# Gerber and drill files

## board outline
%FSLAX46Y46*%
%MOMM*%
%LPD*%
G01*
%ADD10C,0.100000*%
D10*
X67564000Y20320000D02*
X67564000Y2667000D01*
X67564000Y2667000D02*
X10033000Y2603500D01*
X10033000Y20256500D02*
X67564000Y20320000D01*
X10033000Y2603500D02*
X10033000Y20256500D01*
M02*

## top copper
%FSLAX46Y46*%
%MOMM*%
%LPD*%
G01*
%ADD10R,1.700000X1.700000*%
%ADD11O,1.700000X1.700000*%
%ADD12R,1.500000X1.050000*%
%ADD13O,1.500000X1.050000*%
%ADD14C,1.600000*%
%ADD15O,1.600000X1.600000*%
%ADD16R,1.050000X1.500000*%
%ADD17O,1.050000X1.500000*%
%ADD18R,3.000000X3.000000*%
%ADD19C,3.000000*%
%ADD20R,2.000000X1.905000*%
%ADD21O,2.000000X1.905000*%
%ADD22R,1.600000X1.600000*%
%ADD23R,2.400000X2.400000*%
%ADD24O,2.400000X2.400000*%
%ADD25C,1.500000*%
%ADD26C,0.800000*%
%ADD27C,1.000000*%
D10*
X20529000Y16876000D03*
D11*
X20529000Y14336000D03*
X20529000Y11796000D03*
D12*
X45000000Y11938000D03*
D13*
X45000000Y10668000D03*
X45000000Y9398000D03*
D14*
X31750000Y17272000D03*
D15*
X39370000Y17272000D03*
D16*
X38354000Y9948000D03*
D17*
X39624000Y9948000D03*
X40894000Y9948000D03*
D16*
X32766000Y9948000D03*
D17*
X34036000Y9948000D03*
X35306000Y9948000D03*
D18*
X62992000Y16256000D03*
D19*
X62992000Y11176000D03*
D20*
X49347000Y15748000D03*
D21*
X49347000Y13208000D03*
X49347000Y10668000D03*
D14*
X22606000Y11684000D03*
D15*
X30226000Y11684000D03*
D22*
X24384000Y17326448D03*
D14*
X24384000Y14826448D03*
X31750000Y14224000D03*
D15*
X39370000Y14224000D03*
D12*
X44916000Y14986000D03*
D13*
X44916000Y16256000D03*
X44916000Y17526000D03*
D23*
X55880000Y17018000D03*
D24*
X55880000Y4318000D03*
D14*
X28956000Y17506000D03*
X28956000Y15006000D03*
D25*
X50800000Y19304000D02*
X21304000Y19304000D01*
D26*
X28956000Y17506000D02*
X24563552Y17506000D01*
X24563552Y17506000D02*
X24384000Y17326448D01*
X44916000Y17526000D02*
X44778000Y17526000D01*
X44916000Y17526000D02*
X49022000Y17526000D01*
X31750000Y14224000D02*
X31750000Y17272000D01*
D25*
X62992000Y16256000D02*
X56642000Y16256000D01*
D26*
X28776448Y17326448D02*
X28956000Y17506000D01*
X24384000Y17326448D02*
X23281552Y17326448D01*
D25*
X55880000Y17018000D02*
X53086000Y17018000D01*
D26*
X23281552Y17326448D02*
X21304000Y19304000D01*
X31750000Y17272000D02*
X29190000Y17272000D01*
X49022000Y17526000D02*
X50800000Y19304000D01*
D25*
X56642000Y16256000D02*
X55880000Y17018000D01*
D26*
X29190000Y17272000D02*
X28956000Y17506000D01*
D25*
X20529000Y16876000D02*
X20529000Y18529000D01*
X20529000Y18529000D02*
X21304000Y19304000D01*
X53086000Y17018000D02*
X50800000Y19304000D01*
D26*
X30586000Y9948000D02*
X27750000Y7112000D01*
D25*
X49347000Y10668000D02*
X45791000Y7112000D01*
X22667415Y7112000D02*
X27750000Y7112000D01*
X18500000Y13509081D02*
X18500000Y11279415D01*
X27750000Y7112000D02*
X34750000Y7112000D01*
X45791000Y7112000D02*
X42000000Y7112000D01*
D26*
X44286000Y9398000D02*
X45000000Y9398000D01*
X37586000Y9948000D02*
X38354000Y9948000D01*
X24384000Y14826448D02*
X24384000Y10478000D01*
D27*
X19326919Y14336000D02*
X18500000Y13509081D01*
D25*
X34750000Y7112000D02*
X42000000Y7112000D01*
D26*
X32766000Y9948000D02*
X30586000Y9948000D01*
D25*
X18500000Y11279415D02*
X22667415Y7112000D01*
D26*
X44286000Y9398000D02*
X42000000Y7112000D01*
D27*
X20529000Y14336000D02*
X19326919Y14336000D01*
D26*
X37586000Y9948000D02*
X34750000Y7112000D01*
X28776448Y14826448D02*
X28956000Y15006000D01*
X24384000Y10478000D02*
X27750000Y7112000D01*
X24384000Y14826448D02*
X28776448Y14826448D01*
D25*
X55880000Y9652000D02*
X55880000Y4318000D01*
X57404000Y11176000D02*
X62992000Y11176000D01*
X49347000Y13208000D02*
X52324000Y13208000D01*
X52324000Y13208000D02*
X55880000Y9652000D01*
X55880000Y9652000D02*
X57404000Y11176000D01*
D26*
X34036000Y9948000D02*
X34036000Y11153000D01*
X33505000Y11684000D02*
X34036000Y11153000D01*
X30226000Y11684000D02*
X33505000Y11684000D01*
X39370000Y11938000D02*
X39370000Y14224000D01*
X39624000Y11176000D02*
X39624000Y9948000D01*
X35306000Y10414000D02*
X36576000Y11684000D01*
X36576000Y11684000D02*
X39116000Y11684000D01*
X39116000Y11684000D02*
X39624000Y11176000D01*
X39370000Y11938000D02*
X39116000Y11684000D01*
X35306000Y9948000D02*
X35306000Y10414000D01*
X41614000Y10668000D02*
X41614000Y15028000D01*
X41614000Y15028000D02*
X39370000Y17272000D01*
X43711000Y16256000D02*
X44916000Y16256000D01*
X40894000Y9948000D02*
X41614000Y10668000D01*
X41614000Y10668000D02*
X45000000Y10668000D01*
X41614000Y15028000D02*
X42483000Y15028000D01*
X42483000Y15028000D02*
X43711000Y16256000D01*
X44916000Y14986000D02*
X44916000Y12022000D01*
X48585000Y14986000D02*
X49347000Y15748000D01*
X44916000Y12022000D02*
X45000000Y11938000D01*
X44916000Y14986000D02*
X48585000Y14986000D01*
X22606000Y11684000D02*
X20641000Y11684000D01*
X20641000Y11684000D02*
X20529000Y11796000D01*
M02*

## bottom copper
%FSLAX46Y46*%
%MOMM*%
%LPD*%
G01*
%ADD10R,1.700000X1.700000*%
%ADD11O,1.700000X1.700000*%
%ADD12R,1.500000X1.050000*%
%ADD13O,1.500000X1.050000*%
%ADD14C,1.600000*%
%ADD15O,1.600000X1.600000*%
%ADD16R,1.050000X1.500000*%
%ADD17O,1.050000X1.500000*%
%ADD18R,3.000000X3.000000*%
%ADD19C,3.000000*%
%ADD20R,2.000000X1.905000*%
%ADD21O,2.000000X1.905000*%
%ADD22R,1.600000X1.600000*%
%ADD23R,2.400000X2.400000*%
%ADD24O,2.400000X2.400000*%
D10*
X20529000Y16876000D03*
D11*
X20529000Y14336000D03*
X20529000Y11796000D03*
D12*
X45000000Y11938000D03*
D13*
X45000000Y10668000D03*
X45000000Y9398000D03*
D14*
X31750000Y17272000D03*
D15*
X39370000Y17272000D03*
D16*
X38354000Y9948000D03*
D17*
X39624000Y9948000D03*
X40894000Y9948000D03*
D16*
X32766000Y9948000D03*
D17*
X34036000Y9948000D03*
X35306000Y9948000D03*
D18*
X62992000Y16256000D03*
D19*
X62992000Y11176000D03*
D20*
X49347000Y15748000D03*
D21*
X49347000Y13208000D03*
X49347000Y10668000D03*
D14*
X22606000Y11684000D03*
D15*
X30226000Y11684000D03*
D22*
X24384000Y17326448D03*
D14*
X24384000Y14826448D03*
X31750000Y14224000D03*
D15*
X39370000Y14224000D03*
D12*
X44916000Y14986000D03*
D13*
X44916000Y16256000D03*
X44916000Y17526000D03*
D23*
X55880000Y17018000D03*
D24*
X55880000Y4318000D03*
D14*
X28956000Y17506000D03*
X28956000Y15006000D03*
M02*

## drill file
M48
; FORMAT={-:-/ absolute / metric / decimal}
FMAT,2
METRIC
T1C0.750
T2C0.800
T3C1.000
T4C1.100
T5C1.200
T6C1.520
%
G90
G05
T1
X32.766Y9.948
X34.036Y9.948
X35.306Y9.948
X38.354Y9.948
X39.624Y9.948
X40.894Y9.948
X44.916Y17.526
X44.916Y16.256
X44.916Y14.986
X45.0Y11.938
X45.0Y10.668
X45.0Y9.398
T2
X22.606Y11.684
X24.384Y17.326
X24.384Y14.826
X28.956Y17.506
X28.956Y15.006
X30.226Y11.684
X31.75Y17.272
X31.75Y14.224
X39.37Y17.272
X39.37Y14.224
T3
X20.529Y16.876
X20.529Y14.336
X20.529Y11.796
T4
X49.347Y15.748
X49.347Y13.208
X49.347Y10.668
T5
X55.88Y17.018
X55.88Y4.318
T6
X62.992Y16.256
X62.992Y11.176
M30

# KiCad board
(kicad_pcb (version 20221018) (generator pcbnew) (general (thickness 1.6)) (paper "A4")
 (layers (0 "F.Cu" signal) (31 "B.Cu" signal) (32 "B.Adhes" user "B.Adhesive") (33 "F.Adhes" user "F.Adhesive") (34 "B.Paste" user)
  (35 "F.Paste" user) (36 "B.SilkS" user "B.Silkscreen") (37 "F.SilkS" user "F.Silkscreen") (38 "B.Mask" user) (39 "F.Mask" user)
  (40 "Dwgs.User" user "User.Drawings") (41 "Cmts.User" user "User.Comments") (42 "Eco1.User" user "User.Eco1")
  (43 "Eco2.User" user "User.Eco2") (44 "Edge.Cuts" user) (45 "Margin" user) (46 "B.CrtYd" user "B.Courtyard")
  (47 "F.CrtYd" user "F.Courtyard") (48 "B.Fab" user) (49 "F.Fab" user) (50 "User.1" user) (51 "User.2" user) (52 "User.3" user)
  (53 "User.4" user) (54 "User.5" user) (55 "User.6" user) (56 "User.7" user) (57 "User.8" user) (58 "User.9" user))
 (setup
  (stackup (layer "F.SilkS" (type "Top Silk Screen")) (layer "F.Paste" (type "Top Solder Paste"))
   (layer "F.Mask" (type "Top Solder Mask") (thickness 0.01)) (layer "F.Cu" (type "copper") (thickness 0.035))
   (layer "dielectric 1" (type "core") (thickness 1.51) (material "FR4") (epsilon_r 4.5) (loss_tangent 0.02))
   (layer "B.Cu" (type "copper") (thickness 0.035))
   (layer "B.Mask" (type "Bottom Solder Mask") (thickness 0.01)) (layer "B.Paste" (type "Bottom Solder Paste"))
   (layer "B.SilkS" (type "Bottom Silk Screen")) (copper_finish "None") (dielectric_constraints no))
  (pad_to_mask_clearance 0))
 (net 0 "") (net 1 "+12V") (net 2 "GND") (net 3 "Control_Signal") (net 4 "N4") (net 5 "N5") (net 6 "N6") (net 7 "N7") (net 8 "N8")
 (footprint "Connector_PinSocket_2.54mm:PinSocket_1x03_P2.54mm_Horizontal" (layer "F.Cu") (at 20.529 -16.876)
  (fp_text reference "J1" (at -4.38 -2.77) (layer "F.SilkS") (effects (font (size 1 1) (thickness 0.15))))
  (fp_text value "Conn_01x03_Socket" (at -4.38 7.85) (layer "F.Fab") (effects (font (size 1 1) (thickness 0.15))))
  (pad "1" thru_hole rect (at 0 0) (size 1.7 1.7) (drill 1) (layers "*.Cu" "*.Mask") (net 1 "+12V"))
  (pad "2" thru_hole oval (at 0 2.54) (size 1.7 1.7) (drill 1) (layers "*.Cu" "*.Mask") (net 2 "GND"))
  (pad "3" thru_hole oval (at 0 5.08) (size 1.7 1.7) (drill 1) (layers "*.Cu" "*.Mask") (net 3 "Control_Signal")))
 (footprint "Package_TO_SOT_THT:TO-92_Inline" (layer "F.Cu") (at 45 -11.938 -90)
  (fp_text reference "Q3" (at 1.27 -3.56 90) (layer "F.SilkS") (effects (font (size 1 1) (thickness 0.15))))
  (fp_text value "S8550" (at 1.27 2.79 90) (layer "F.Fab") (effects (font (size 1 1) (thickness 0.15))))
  (pad "1" thru_hole rect (at 0 0 270) (size 1.05 1.5) (drill 0.75) (layers "*.Cu" "*.Mask") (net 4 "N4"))
  (pad "2" thru_hole oval (at 1.27 0 270) (size 1.05 1.5) (drill 0.75) (layers "*.Cu" "*.Mask") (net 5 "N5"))
  (pad "3" thru_hole oval (at 2.54 0 270) (size 1.05 1.5) (drill 0.75) (layers "*.Cu" "*.Mask") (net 2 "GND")))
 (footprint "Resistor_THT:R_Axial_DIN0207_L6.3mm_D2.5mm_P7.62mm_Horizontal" (layer "F.Cu") (at 31.75 -17.272)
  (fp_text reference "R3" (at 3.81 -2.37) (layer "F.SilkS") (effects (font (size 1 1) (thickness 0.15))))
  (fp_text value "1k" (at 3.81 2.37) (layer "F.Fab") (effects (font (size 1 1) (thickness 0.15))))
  (pad "1" thru_hole circle (at 0 0) (size 1.6 1.6) (drill 0.8) (layers "*.Cu" "*.Mask") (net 1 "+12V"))
  (pad "2" thru_hole oval (at 7.62 0) (size 1.6 1.6) (drill 0.8) (layers "*.Cu" "*.Mask") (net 5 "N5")))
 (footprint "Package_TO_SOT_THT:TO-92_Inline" (layer "F.Cu") (at 38.354 -9.948)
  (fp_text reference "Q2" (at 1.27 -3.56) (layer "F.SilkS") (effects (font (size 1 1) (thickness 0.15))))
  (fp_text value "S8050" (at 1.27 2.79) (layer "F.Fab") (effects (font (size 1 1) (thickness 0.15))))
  (pad "1" thru_hole rect (at 0 0) (size 1.05 1.5) (drill 0.75) (layers "*.Cu" "*.Mask") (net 2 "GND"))
  (pad "2" thru_hole oval (at 1.27 0) (size 1.05 1.5) (drill 0.75) (layers "*.Cu" "*.Mask") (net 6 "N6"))
  (pad "3" thru_hole oval (at 2.54 0) (size 1.05 1.5) (drill 0.75) (layers "*.Cu" "*.Mask") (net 5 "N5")))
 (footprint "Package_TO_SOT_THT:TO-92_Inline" (layer "F.Cu") (at 32.766 -9.948)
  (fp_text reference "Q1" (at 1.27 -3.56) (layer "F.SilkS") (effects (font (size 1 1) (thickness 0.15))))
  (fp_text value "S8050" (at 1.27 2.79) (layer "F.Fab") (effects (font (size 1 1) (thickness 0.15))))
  (pad "1" thru_hole rect (at 0 0) (size 1.05 1.5) (drill 0.75) (layers "*.Cu" "*.Mask") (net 2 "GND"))
  (pad "2" thru_hole oval (at 1.27 0) (size 1.05 1.5) (drill 0.75) (layers "*.Cu" "*.Mask") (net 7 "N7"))
  (pad "3" thru_hole oval (at 2.54 0) (size 1.05 1.5) (drill 0.75) (layers "*.Cu" "*.Mask") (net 6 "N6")))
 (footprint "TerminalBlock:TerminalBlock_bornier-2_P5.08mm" (layer "F.Cu") (at 62.992 -16.256 -90)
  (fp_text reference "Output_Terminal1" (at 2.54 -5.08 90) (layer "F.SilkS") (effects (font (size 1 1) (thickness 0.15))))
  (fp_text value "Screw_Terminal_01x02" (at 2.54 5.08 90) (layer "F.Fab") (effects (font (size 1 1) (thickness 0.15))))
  (pad "1" thru_hole rect (at 0 0 270) (size 3 3) (drill 1.52) (layers "*.Cu" "*.Mask") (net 1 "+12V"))
  (pad "2" thru_hole circle (at 5.08 0 270) (size 3 3) (drill 1.52) (layers "*.Cu" "*.Mask") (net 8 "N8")))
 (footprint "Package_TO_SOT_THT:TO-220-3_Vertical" (layer "F.Cu") (at 49.347 -15.748 -90)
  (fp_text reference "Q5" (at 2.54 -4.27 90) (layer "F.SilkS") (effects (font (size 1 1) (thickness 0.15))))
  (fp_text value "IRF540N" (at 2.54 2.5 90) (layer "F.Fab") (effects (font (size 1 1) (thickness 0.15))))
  (pad "1" thru_hole rect (at 0 0 270) (size 1.905 2) (drill 1.1) (layers "*.Cu" "*.Mask") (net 4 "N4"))
  (pad "2" thru_hole oval (at 2.54 0 270) (size 1.905 2) (drill 1.1) (layers "*.Cu" "*.Mask") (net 8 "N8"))
  (pad "3" thru_hole oval (at 5.08 0 270) (size 1.905 2) (drill 1.1) (layers "*.Cu" "*.Mask") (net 2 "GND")))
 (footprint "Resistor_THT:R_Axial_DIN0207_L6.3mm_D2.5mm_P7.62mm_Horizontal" (layer "F.Cu") (at 22.606 -11.684)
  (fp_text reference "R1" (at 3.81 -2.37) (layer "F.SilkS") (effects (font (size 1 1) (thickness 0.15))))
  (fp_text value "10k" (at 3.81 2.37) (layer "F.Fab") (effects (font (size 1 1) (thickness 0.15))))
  (pad "1" thru_hole circle (at 0 0) (size 1.6 1.6) (drill 0.8) (layers "*.Cu" "*.Mask") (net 3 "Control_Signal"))
  (pad "2" thru_hole oval (at 7.62 0) (size 1.6 1.6) (drill 0.8) (layers "*.Cu" "*.Mask") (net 7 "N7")))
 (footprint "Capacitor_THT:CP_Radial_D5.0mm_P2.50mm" (layer "F.Cu") (at 24.384 -17.326448 -90)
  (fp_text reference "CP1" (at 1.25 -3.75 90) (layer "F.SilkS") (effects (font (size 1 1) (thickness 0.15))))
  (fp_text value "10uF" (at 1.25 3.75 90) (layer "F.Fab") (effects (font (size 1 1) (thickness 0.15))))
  (pad "1" thru_hole rect (at 0 0 270) (size 1.6 1.6) (drill 0.8) (layers "*.Cu" "*.Mask") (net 1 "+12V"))
  (pad "2" thru_hole circle (at 2.5 0 270) (size 1.6 1.6) (drill 0.8) (layers "*.Cu" "*.Mask") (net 2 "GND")))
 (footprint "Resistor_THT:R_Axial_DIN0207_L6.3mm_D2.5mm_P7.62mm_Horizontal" (layer "F.Cu") (at 31.75 -14.224)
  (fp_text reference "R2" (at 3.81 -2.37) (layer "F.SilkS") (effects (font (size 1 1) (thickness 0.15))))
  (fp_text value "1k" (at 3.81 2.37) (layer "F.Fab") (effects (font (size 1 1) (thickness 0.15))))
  (pad "1" thru_hole circle (at 0 0) (size 1.6 1.6) (drill 0.8) (layers "*.Cu" "*.Mask") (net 1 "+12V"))
  (pad "2" thru_hole oval (at 7.62 0) (size 1.6 1.6) (drill 0.8) (layers "*.Cu" "*.Mask") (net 6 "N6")))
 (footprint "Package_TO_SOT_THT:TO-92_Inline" (layer "F.Cu") (at 44.916 -14.986 90)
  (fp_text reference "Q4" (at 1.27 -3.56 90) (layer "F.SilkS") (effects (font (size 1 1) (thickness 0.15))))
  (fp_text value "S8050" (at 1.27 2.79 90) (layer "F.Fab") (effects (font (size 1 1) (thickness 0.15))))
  (pad "1" thru_hole rect (at 0 0 90) (size 1.05 1.5) (drill 0.75) (layers "*.Cu" "*.Mask") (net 4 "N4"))
  (pad "2" thru_hole oval (at 1.27 0 90) (size 1.05 1.5) (drill 0.75) (layers "*.Cu" "*.Mask") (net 5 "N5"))
  (pad "3" thru_hole oval (at 2.54 0 90) (size 1.05 1.5) (drill 0.75) (layers "*.Cu" "*.Mask") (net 1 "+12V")))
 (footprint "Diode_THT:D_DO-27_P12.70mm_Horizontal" (layer "F.Cu") (at 55.88 -17.018 -90)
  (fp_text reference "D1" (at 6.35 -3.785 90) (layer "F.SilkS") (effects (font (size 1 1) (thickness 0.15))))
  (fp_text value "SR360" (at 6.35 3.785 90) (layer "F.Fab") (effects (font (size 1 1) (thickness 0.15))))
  (pad "1" thru_hole rect (at 0 0 270) (size 2.4 2.4) (drill 1.2) (layers "*.Cu" "*.Mask") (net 1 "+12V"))
  (pad "2" thru_hole oval (at 12.7 0 270) (size 2.4 2.4) (drill 1.2) (layers "*.Cu" "*.Mask") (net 8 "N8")))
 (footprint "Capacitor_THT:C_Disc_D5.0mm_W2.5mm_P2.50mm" (layer "F.Cu") (at 28.956 -17.506 -90)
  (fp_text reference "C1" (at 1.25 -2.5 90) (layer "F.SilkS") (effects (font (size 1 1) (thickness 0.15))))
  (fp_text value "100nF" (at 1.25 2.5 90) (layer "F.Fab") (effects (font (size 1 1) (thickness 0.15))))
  (pad "1" thru_hole circle (at 0 0 270) (size 1.6 1.6) (drill 0.8) (layers "*.Cu" "*.Mask") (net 1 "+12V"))
  (pad "2" thru_hole circle (at 2.5 0 270) (size 1.6 1.6) (drill 0.8) (layers "*.Cu" "*.Mask") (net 2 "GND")))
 (gr_line (start 67.564 -20.32) (end 67.564 -2.667) (stroke (width 0.1) (type solid)) (layer "Edge.Cuts"))
 (gr_line (start 67.564 -2.667) (end 10.033 -2.6035) (stroke (width 0.1) (type solid)) (layer "Edge.Cuts"))
 (gr_line (start 10.033 -20.2565) (end 67.564 -20.32) (stroke (width 0.1) (type solid)) (layer "Edge.Cuts"))
 (gr_line (start 10.033 -2.6035) (end 10.033 -20.2565) (stroke (width 0.1) (type solid)) (layer "Edge.Cuts"))
 (segment (start 50.8 -19.304) (end 21.304 -19.304) (width 1.5) (layer "F.Cu") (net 1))
 (segment (start 28.956 -17.506) (end 24.563552 -17.506) (width 0.8) (layer "F.Cu") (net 1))
 (segment (start 24.563552 -17.506) (end 24.384 -17.326448) (width 0.8) (layer "F.Cu") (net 1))
 (segment (start 44.916 -17.526) (end 44.778 -17.526) (width 0.8) (layer "F.Cu") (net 1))
 (segment (start 44.916 -17.526) (end 49.022 -17.526) (width 0.8) (layer "F.Cu") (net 1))
 (segment (start 31.75 -14.224) (end 31.75 -17.272) (width 0.8) (layer "F.Cu") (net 1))
 (segment (start 62.992 -16.256) (end 56.642 -16.256) (width 1.5) (layer "F.Cu") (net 1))
 (segment (start 28.776448 -17.326448) (end 28.956 -17.506) (width 0.8) (layer "F.Cu") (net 1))
 (segment (start 24.384 -17.326448) (end 23.281552 -17.326448) (width 0.8) (layer "F.Cu") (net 1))
 (segment (start 55.88 -17.018) (end 53.086 -17.018) (width 1.5) (layer "F.Cu") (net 1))
 (segment (start 23.281552 -17.326448) (end 21.304 -19.304) (width 0.8) (layer "F.Cu") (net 1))
 (segment (start 31.75 -17.272) (end 29.19 -17.272) (width 0.8) (layer "F.Cu") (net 1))
 (segment (start 49.022 -17.526) (end 50.8 -19.304) (width 0.8) (layer "F.Cu") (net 1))
 (segment (start 56.642 -16.256) (end 55.88 -17.018) (width 1.5) (layer "F.Cu") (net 1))
 (segment (start 29.19 -17.272) (end 28.956 -17.506) (width 0.8) (layer "F.Cu") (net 1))
 (segment (start 20.529 -16.876) (end 20.529 -18.529) (width 1.5) (layer "F.Cu") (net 1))
 (segment (start 20.529 -18.529) (end 21.304 -19.304) (width 1.5) (layer "F.Cu") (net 1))
 (segment (start 53.086 -17.018) (end 50.8 -19.304) (width 1.5) (layer "F.Cu") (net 1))
 (segment (start 30.586 -9.948) (end 27.75 -7.112) (width 0.8) (layer "F.Cu") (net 2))
 (segment (start 49.347 -10.668) (end 45.791 -7.112) (width 1.5) (layer "F.Cu") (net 2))
 (segment (start 22.667415 -7.112) (end 27.75 -7.112) (width 1.5) (layer "F.Cu") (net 2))
 (segment (start 18.5 -13.509081) (end 18.5 -11.279415) (width 1.5) (layer "F.Cu") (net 2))
 (segment (start 27.75 -7.112) (end 34.75 -7.112) (width 1.5) (layer "F.Cu") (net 2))
 (segment (start 45.791 -7.112) (end 42 -7.112) (width 1.5) (layer "F.Cu") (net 2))
 (segment (start 44.286 -9.398) (end 45 -9.398) (width 0.8) (layer "F.Cu") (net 2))
 (segment (start 37.586 -9.948) (end 38.354 -9.948) (width 0.8) (layer "F.Cu") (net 2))
 (segment (start 24.384 -14.826448) (end 24.384 -10.478) (width 0.8) (layer "F.Cu") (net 2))
 (segment (start 19.326919 -14.336) (end 18.5 -13.509081) (width 1) (layer "F.Cu") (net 2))
 (segment (start 34.75 -7.112) (end 42 -7.112) (width 1.5) (layer "F.Cu") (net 2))
 (segment (start 32.766 -9.948) (end 30.586 -9.948) (width 0.8) (layer "F.Cu") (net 2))
 (segment (start 18.5 -11.279415) (end 22.667415 -7.112) (width 1.5) (layer "F.Cu") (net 2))
 (segment (start 44.286 -9.398) (end 42 -7.112) (width 0.8) (layer "F.Cu") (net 2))
 (segment (start 20.529 -14.336) (end 19.326919 -14.336) (width 1) (layer "F.Cu") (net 2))
 (segment (start 37.586 -9.948) (end 34.75 -7.112) (width 0.8) (layer "F.Cu") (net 2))
 (segment (start 28.776448 -14.826448) (end 28.956 -15.006) (width 0.8) (layer "F.Cu") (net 2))
 (segment (start 24.384 -10.478) (end 27.75 -7.112) (width 0.8) (layer "F.Cu") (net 2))
 (segment (start 24.384 -14.826448) (end 28.776448 -14.826448) (width 0.8) (layer "F.Cu") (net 2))
 (segment (start 55.88 -9.652) (end 55.88 -4.318) (width 1.5) (layer "F.Cu") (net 8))
 (segment (start 57.404 -11.176) (end 62.992 -11.176) (width 1.5) (layer "F.Cu") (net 8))
 (segment (start 49.347 -13.208) (end 52.324 -13.208) (width 1.5) (layer "F.Cu") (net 8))
 (segment (start 52.324 -13.208) (end 55.88 -9.652) (width 1.5) (layer "F.Cu") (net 8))
 (segment (start 55.88 -9.652) (end 57.404 -11.176) (width 1.5) (layer "F.Cu") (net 8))
 (segment (start 34.036 -9.948) (end 34.036 -11.153) (width 0.8) (layer "F.Cu") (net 7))
 (segment (start 33.505 -11.684) (end 34.036 -11.153) (width 0.8) (layer "F.Cu") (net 7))
 (segment (start 30.226 -11.684) (end 33.505 -11.684) (width 0.8) (layer "F.Cu") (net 7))
 (segment (start 39.37 -11.938) (end 39.37 -14.224) (width 0.8) (layer "F.Cu") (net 6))
 (segment (start 39.624 -11.176) (end 39.624 -9.948) (width 0.8) (layer "F.Cu") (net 6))
 (segment (start 35.306 -10.414) (end 36.576 -11.684) (width 0.8) (layer "F.Cu") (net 6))
 (segment (start 36.576 -11.684) (end 39.116 -11.684) (width 0.8) (layer "F.Cu") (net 6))
 (segment (start 39.116 -11.684) (end 39.624 -11.176) (width 0.8) (layer "F.Cu") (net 6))
 (segment (start 39.37 -11.938) (end 39.116 -11.684) (width 0.8) (layer "F.Cu") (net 6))
 (segment (start 35.306 -9.948) (end 35.306 -10.414) (width 0.8) (layer "F.Cu") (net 6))
 (segment (start 41.614 -10.668) (end 41.614 -15.028) (width 0.8) (layer "F.Cu") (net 5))
 (segment (start 41.614 -15.028) (end 39.37 -17.272) (width 0.8) (layer "F.Cu") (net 5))
 (segment (start 43.711 -16.256) (end 44.916 -16.256) (width 0.8) (layer "F.Cu") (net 5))
 (segment (start 40.894 -9.948) (end 41.614 -10.668) (width 0.8) (layer "F.Cu") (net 5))
 (segment (start 41.614 -10.668) (end 45 -10.668) (width 0.8) (layer "F.Cu") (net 5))
 (segment (start 41.614 -15.028) (end 42.483 -15.028) (width 0.8) (layer "F.Cu") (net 5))
 (segment (start 42.483 -15.028) (end 43.711 -16.256) (width 0.8) (layer "F.Cu") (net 5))
 (segment (start 44.916 -14.986) (end 44.916 -12.022) (width 0.8) (layer "F.Cu") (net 4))
 (segment (start 48.585 -14.986) (end 49.347 -15.748) (width 0.8) (layer "F.Cu") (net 4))
 (segment (start 44.916 -12.022) (end 45 -11.938) (width 0.8) (layer "F.Cu") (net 4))
 (segment (start 44.916 -14.986) (end 48.585 -14.986) (width 0.8) (layer "F.Cu") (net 4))
 (segment (start 22.606 -11.684) (end 20.641 -11.684) (width 0.8) (layer "F.Cu") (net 3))
 (segment (start 20.641 -11.684) (end 20.529 -11.796) (width 0.8) (layer "F.Cu") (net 3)))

